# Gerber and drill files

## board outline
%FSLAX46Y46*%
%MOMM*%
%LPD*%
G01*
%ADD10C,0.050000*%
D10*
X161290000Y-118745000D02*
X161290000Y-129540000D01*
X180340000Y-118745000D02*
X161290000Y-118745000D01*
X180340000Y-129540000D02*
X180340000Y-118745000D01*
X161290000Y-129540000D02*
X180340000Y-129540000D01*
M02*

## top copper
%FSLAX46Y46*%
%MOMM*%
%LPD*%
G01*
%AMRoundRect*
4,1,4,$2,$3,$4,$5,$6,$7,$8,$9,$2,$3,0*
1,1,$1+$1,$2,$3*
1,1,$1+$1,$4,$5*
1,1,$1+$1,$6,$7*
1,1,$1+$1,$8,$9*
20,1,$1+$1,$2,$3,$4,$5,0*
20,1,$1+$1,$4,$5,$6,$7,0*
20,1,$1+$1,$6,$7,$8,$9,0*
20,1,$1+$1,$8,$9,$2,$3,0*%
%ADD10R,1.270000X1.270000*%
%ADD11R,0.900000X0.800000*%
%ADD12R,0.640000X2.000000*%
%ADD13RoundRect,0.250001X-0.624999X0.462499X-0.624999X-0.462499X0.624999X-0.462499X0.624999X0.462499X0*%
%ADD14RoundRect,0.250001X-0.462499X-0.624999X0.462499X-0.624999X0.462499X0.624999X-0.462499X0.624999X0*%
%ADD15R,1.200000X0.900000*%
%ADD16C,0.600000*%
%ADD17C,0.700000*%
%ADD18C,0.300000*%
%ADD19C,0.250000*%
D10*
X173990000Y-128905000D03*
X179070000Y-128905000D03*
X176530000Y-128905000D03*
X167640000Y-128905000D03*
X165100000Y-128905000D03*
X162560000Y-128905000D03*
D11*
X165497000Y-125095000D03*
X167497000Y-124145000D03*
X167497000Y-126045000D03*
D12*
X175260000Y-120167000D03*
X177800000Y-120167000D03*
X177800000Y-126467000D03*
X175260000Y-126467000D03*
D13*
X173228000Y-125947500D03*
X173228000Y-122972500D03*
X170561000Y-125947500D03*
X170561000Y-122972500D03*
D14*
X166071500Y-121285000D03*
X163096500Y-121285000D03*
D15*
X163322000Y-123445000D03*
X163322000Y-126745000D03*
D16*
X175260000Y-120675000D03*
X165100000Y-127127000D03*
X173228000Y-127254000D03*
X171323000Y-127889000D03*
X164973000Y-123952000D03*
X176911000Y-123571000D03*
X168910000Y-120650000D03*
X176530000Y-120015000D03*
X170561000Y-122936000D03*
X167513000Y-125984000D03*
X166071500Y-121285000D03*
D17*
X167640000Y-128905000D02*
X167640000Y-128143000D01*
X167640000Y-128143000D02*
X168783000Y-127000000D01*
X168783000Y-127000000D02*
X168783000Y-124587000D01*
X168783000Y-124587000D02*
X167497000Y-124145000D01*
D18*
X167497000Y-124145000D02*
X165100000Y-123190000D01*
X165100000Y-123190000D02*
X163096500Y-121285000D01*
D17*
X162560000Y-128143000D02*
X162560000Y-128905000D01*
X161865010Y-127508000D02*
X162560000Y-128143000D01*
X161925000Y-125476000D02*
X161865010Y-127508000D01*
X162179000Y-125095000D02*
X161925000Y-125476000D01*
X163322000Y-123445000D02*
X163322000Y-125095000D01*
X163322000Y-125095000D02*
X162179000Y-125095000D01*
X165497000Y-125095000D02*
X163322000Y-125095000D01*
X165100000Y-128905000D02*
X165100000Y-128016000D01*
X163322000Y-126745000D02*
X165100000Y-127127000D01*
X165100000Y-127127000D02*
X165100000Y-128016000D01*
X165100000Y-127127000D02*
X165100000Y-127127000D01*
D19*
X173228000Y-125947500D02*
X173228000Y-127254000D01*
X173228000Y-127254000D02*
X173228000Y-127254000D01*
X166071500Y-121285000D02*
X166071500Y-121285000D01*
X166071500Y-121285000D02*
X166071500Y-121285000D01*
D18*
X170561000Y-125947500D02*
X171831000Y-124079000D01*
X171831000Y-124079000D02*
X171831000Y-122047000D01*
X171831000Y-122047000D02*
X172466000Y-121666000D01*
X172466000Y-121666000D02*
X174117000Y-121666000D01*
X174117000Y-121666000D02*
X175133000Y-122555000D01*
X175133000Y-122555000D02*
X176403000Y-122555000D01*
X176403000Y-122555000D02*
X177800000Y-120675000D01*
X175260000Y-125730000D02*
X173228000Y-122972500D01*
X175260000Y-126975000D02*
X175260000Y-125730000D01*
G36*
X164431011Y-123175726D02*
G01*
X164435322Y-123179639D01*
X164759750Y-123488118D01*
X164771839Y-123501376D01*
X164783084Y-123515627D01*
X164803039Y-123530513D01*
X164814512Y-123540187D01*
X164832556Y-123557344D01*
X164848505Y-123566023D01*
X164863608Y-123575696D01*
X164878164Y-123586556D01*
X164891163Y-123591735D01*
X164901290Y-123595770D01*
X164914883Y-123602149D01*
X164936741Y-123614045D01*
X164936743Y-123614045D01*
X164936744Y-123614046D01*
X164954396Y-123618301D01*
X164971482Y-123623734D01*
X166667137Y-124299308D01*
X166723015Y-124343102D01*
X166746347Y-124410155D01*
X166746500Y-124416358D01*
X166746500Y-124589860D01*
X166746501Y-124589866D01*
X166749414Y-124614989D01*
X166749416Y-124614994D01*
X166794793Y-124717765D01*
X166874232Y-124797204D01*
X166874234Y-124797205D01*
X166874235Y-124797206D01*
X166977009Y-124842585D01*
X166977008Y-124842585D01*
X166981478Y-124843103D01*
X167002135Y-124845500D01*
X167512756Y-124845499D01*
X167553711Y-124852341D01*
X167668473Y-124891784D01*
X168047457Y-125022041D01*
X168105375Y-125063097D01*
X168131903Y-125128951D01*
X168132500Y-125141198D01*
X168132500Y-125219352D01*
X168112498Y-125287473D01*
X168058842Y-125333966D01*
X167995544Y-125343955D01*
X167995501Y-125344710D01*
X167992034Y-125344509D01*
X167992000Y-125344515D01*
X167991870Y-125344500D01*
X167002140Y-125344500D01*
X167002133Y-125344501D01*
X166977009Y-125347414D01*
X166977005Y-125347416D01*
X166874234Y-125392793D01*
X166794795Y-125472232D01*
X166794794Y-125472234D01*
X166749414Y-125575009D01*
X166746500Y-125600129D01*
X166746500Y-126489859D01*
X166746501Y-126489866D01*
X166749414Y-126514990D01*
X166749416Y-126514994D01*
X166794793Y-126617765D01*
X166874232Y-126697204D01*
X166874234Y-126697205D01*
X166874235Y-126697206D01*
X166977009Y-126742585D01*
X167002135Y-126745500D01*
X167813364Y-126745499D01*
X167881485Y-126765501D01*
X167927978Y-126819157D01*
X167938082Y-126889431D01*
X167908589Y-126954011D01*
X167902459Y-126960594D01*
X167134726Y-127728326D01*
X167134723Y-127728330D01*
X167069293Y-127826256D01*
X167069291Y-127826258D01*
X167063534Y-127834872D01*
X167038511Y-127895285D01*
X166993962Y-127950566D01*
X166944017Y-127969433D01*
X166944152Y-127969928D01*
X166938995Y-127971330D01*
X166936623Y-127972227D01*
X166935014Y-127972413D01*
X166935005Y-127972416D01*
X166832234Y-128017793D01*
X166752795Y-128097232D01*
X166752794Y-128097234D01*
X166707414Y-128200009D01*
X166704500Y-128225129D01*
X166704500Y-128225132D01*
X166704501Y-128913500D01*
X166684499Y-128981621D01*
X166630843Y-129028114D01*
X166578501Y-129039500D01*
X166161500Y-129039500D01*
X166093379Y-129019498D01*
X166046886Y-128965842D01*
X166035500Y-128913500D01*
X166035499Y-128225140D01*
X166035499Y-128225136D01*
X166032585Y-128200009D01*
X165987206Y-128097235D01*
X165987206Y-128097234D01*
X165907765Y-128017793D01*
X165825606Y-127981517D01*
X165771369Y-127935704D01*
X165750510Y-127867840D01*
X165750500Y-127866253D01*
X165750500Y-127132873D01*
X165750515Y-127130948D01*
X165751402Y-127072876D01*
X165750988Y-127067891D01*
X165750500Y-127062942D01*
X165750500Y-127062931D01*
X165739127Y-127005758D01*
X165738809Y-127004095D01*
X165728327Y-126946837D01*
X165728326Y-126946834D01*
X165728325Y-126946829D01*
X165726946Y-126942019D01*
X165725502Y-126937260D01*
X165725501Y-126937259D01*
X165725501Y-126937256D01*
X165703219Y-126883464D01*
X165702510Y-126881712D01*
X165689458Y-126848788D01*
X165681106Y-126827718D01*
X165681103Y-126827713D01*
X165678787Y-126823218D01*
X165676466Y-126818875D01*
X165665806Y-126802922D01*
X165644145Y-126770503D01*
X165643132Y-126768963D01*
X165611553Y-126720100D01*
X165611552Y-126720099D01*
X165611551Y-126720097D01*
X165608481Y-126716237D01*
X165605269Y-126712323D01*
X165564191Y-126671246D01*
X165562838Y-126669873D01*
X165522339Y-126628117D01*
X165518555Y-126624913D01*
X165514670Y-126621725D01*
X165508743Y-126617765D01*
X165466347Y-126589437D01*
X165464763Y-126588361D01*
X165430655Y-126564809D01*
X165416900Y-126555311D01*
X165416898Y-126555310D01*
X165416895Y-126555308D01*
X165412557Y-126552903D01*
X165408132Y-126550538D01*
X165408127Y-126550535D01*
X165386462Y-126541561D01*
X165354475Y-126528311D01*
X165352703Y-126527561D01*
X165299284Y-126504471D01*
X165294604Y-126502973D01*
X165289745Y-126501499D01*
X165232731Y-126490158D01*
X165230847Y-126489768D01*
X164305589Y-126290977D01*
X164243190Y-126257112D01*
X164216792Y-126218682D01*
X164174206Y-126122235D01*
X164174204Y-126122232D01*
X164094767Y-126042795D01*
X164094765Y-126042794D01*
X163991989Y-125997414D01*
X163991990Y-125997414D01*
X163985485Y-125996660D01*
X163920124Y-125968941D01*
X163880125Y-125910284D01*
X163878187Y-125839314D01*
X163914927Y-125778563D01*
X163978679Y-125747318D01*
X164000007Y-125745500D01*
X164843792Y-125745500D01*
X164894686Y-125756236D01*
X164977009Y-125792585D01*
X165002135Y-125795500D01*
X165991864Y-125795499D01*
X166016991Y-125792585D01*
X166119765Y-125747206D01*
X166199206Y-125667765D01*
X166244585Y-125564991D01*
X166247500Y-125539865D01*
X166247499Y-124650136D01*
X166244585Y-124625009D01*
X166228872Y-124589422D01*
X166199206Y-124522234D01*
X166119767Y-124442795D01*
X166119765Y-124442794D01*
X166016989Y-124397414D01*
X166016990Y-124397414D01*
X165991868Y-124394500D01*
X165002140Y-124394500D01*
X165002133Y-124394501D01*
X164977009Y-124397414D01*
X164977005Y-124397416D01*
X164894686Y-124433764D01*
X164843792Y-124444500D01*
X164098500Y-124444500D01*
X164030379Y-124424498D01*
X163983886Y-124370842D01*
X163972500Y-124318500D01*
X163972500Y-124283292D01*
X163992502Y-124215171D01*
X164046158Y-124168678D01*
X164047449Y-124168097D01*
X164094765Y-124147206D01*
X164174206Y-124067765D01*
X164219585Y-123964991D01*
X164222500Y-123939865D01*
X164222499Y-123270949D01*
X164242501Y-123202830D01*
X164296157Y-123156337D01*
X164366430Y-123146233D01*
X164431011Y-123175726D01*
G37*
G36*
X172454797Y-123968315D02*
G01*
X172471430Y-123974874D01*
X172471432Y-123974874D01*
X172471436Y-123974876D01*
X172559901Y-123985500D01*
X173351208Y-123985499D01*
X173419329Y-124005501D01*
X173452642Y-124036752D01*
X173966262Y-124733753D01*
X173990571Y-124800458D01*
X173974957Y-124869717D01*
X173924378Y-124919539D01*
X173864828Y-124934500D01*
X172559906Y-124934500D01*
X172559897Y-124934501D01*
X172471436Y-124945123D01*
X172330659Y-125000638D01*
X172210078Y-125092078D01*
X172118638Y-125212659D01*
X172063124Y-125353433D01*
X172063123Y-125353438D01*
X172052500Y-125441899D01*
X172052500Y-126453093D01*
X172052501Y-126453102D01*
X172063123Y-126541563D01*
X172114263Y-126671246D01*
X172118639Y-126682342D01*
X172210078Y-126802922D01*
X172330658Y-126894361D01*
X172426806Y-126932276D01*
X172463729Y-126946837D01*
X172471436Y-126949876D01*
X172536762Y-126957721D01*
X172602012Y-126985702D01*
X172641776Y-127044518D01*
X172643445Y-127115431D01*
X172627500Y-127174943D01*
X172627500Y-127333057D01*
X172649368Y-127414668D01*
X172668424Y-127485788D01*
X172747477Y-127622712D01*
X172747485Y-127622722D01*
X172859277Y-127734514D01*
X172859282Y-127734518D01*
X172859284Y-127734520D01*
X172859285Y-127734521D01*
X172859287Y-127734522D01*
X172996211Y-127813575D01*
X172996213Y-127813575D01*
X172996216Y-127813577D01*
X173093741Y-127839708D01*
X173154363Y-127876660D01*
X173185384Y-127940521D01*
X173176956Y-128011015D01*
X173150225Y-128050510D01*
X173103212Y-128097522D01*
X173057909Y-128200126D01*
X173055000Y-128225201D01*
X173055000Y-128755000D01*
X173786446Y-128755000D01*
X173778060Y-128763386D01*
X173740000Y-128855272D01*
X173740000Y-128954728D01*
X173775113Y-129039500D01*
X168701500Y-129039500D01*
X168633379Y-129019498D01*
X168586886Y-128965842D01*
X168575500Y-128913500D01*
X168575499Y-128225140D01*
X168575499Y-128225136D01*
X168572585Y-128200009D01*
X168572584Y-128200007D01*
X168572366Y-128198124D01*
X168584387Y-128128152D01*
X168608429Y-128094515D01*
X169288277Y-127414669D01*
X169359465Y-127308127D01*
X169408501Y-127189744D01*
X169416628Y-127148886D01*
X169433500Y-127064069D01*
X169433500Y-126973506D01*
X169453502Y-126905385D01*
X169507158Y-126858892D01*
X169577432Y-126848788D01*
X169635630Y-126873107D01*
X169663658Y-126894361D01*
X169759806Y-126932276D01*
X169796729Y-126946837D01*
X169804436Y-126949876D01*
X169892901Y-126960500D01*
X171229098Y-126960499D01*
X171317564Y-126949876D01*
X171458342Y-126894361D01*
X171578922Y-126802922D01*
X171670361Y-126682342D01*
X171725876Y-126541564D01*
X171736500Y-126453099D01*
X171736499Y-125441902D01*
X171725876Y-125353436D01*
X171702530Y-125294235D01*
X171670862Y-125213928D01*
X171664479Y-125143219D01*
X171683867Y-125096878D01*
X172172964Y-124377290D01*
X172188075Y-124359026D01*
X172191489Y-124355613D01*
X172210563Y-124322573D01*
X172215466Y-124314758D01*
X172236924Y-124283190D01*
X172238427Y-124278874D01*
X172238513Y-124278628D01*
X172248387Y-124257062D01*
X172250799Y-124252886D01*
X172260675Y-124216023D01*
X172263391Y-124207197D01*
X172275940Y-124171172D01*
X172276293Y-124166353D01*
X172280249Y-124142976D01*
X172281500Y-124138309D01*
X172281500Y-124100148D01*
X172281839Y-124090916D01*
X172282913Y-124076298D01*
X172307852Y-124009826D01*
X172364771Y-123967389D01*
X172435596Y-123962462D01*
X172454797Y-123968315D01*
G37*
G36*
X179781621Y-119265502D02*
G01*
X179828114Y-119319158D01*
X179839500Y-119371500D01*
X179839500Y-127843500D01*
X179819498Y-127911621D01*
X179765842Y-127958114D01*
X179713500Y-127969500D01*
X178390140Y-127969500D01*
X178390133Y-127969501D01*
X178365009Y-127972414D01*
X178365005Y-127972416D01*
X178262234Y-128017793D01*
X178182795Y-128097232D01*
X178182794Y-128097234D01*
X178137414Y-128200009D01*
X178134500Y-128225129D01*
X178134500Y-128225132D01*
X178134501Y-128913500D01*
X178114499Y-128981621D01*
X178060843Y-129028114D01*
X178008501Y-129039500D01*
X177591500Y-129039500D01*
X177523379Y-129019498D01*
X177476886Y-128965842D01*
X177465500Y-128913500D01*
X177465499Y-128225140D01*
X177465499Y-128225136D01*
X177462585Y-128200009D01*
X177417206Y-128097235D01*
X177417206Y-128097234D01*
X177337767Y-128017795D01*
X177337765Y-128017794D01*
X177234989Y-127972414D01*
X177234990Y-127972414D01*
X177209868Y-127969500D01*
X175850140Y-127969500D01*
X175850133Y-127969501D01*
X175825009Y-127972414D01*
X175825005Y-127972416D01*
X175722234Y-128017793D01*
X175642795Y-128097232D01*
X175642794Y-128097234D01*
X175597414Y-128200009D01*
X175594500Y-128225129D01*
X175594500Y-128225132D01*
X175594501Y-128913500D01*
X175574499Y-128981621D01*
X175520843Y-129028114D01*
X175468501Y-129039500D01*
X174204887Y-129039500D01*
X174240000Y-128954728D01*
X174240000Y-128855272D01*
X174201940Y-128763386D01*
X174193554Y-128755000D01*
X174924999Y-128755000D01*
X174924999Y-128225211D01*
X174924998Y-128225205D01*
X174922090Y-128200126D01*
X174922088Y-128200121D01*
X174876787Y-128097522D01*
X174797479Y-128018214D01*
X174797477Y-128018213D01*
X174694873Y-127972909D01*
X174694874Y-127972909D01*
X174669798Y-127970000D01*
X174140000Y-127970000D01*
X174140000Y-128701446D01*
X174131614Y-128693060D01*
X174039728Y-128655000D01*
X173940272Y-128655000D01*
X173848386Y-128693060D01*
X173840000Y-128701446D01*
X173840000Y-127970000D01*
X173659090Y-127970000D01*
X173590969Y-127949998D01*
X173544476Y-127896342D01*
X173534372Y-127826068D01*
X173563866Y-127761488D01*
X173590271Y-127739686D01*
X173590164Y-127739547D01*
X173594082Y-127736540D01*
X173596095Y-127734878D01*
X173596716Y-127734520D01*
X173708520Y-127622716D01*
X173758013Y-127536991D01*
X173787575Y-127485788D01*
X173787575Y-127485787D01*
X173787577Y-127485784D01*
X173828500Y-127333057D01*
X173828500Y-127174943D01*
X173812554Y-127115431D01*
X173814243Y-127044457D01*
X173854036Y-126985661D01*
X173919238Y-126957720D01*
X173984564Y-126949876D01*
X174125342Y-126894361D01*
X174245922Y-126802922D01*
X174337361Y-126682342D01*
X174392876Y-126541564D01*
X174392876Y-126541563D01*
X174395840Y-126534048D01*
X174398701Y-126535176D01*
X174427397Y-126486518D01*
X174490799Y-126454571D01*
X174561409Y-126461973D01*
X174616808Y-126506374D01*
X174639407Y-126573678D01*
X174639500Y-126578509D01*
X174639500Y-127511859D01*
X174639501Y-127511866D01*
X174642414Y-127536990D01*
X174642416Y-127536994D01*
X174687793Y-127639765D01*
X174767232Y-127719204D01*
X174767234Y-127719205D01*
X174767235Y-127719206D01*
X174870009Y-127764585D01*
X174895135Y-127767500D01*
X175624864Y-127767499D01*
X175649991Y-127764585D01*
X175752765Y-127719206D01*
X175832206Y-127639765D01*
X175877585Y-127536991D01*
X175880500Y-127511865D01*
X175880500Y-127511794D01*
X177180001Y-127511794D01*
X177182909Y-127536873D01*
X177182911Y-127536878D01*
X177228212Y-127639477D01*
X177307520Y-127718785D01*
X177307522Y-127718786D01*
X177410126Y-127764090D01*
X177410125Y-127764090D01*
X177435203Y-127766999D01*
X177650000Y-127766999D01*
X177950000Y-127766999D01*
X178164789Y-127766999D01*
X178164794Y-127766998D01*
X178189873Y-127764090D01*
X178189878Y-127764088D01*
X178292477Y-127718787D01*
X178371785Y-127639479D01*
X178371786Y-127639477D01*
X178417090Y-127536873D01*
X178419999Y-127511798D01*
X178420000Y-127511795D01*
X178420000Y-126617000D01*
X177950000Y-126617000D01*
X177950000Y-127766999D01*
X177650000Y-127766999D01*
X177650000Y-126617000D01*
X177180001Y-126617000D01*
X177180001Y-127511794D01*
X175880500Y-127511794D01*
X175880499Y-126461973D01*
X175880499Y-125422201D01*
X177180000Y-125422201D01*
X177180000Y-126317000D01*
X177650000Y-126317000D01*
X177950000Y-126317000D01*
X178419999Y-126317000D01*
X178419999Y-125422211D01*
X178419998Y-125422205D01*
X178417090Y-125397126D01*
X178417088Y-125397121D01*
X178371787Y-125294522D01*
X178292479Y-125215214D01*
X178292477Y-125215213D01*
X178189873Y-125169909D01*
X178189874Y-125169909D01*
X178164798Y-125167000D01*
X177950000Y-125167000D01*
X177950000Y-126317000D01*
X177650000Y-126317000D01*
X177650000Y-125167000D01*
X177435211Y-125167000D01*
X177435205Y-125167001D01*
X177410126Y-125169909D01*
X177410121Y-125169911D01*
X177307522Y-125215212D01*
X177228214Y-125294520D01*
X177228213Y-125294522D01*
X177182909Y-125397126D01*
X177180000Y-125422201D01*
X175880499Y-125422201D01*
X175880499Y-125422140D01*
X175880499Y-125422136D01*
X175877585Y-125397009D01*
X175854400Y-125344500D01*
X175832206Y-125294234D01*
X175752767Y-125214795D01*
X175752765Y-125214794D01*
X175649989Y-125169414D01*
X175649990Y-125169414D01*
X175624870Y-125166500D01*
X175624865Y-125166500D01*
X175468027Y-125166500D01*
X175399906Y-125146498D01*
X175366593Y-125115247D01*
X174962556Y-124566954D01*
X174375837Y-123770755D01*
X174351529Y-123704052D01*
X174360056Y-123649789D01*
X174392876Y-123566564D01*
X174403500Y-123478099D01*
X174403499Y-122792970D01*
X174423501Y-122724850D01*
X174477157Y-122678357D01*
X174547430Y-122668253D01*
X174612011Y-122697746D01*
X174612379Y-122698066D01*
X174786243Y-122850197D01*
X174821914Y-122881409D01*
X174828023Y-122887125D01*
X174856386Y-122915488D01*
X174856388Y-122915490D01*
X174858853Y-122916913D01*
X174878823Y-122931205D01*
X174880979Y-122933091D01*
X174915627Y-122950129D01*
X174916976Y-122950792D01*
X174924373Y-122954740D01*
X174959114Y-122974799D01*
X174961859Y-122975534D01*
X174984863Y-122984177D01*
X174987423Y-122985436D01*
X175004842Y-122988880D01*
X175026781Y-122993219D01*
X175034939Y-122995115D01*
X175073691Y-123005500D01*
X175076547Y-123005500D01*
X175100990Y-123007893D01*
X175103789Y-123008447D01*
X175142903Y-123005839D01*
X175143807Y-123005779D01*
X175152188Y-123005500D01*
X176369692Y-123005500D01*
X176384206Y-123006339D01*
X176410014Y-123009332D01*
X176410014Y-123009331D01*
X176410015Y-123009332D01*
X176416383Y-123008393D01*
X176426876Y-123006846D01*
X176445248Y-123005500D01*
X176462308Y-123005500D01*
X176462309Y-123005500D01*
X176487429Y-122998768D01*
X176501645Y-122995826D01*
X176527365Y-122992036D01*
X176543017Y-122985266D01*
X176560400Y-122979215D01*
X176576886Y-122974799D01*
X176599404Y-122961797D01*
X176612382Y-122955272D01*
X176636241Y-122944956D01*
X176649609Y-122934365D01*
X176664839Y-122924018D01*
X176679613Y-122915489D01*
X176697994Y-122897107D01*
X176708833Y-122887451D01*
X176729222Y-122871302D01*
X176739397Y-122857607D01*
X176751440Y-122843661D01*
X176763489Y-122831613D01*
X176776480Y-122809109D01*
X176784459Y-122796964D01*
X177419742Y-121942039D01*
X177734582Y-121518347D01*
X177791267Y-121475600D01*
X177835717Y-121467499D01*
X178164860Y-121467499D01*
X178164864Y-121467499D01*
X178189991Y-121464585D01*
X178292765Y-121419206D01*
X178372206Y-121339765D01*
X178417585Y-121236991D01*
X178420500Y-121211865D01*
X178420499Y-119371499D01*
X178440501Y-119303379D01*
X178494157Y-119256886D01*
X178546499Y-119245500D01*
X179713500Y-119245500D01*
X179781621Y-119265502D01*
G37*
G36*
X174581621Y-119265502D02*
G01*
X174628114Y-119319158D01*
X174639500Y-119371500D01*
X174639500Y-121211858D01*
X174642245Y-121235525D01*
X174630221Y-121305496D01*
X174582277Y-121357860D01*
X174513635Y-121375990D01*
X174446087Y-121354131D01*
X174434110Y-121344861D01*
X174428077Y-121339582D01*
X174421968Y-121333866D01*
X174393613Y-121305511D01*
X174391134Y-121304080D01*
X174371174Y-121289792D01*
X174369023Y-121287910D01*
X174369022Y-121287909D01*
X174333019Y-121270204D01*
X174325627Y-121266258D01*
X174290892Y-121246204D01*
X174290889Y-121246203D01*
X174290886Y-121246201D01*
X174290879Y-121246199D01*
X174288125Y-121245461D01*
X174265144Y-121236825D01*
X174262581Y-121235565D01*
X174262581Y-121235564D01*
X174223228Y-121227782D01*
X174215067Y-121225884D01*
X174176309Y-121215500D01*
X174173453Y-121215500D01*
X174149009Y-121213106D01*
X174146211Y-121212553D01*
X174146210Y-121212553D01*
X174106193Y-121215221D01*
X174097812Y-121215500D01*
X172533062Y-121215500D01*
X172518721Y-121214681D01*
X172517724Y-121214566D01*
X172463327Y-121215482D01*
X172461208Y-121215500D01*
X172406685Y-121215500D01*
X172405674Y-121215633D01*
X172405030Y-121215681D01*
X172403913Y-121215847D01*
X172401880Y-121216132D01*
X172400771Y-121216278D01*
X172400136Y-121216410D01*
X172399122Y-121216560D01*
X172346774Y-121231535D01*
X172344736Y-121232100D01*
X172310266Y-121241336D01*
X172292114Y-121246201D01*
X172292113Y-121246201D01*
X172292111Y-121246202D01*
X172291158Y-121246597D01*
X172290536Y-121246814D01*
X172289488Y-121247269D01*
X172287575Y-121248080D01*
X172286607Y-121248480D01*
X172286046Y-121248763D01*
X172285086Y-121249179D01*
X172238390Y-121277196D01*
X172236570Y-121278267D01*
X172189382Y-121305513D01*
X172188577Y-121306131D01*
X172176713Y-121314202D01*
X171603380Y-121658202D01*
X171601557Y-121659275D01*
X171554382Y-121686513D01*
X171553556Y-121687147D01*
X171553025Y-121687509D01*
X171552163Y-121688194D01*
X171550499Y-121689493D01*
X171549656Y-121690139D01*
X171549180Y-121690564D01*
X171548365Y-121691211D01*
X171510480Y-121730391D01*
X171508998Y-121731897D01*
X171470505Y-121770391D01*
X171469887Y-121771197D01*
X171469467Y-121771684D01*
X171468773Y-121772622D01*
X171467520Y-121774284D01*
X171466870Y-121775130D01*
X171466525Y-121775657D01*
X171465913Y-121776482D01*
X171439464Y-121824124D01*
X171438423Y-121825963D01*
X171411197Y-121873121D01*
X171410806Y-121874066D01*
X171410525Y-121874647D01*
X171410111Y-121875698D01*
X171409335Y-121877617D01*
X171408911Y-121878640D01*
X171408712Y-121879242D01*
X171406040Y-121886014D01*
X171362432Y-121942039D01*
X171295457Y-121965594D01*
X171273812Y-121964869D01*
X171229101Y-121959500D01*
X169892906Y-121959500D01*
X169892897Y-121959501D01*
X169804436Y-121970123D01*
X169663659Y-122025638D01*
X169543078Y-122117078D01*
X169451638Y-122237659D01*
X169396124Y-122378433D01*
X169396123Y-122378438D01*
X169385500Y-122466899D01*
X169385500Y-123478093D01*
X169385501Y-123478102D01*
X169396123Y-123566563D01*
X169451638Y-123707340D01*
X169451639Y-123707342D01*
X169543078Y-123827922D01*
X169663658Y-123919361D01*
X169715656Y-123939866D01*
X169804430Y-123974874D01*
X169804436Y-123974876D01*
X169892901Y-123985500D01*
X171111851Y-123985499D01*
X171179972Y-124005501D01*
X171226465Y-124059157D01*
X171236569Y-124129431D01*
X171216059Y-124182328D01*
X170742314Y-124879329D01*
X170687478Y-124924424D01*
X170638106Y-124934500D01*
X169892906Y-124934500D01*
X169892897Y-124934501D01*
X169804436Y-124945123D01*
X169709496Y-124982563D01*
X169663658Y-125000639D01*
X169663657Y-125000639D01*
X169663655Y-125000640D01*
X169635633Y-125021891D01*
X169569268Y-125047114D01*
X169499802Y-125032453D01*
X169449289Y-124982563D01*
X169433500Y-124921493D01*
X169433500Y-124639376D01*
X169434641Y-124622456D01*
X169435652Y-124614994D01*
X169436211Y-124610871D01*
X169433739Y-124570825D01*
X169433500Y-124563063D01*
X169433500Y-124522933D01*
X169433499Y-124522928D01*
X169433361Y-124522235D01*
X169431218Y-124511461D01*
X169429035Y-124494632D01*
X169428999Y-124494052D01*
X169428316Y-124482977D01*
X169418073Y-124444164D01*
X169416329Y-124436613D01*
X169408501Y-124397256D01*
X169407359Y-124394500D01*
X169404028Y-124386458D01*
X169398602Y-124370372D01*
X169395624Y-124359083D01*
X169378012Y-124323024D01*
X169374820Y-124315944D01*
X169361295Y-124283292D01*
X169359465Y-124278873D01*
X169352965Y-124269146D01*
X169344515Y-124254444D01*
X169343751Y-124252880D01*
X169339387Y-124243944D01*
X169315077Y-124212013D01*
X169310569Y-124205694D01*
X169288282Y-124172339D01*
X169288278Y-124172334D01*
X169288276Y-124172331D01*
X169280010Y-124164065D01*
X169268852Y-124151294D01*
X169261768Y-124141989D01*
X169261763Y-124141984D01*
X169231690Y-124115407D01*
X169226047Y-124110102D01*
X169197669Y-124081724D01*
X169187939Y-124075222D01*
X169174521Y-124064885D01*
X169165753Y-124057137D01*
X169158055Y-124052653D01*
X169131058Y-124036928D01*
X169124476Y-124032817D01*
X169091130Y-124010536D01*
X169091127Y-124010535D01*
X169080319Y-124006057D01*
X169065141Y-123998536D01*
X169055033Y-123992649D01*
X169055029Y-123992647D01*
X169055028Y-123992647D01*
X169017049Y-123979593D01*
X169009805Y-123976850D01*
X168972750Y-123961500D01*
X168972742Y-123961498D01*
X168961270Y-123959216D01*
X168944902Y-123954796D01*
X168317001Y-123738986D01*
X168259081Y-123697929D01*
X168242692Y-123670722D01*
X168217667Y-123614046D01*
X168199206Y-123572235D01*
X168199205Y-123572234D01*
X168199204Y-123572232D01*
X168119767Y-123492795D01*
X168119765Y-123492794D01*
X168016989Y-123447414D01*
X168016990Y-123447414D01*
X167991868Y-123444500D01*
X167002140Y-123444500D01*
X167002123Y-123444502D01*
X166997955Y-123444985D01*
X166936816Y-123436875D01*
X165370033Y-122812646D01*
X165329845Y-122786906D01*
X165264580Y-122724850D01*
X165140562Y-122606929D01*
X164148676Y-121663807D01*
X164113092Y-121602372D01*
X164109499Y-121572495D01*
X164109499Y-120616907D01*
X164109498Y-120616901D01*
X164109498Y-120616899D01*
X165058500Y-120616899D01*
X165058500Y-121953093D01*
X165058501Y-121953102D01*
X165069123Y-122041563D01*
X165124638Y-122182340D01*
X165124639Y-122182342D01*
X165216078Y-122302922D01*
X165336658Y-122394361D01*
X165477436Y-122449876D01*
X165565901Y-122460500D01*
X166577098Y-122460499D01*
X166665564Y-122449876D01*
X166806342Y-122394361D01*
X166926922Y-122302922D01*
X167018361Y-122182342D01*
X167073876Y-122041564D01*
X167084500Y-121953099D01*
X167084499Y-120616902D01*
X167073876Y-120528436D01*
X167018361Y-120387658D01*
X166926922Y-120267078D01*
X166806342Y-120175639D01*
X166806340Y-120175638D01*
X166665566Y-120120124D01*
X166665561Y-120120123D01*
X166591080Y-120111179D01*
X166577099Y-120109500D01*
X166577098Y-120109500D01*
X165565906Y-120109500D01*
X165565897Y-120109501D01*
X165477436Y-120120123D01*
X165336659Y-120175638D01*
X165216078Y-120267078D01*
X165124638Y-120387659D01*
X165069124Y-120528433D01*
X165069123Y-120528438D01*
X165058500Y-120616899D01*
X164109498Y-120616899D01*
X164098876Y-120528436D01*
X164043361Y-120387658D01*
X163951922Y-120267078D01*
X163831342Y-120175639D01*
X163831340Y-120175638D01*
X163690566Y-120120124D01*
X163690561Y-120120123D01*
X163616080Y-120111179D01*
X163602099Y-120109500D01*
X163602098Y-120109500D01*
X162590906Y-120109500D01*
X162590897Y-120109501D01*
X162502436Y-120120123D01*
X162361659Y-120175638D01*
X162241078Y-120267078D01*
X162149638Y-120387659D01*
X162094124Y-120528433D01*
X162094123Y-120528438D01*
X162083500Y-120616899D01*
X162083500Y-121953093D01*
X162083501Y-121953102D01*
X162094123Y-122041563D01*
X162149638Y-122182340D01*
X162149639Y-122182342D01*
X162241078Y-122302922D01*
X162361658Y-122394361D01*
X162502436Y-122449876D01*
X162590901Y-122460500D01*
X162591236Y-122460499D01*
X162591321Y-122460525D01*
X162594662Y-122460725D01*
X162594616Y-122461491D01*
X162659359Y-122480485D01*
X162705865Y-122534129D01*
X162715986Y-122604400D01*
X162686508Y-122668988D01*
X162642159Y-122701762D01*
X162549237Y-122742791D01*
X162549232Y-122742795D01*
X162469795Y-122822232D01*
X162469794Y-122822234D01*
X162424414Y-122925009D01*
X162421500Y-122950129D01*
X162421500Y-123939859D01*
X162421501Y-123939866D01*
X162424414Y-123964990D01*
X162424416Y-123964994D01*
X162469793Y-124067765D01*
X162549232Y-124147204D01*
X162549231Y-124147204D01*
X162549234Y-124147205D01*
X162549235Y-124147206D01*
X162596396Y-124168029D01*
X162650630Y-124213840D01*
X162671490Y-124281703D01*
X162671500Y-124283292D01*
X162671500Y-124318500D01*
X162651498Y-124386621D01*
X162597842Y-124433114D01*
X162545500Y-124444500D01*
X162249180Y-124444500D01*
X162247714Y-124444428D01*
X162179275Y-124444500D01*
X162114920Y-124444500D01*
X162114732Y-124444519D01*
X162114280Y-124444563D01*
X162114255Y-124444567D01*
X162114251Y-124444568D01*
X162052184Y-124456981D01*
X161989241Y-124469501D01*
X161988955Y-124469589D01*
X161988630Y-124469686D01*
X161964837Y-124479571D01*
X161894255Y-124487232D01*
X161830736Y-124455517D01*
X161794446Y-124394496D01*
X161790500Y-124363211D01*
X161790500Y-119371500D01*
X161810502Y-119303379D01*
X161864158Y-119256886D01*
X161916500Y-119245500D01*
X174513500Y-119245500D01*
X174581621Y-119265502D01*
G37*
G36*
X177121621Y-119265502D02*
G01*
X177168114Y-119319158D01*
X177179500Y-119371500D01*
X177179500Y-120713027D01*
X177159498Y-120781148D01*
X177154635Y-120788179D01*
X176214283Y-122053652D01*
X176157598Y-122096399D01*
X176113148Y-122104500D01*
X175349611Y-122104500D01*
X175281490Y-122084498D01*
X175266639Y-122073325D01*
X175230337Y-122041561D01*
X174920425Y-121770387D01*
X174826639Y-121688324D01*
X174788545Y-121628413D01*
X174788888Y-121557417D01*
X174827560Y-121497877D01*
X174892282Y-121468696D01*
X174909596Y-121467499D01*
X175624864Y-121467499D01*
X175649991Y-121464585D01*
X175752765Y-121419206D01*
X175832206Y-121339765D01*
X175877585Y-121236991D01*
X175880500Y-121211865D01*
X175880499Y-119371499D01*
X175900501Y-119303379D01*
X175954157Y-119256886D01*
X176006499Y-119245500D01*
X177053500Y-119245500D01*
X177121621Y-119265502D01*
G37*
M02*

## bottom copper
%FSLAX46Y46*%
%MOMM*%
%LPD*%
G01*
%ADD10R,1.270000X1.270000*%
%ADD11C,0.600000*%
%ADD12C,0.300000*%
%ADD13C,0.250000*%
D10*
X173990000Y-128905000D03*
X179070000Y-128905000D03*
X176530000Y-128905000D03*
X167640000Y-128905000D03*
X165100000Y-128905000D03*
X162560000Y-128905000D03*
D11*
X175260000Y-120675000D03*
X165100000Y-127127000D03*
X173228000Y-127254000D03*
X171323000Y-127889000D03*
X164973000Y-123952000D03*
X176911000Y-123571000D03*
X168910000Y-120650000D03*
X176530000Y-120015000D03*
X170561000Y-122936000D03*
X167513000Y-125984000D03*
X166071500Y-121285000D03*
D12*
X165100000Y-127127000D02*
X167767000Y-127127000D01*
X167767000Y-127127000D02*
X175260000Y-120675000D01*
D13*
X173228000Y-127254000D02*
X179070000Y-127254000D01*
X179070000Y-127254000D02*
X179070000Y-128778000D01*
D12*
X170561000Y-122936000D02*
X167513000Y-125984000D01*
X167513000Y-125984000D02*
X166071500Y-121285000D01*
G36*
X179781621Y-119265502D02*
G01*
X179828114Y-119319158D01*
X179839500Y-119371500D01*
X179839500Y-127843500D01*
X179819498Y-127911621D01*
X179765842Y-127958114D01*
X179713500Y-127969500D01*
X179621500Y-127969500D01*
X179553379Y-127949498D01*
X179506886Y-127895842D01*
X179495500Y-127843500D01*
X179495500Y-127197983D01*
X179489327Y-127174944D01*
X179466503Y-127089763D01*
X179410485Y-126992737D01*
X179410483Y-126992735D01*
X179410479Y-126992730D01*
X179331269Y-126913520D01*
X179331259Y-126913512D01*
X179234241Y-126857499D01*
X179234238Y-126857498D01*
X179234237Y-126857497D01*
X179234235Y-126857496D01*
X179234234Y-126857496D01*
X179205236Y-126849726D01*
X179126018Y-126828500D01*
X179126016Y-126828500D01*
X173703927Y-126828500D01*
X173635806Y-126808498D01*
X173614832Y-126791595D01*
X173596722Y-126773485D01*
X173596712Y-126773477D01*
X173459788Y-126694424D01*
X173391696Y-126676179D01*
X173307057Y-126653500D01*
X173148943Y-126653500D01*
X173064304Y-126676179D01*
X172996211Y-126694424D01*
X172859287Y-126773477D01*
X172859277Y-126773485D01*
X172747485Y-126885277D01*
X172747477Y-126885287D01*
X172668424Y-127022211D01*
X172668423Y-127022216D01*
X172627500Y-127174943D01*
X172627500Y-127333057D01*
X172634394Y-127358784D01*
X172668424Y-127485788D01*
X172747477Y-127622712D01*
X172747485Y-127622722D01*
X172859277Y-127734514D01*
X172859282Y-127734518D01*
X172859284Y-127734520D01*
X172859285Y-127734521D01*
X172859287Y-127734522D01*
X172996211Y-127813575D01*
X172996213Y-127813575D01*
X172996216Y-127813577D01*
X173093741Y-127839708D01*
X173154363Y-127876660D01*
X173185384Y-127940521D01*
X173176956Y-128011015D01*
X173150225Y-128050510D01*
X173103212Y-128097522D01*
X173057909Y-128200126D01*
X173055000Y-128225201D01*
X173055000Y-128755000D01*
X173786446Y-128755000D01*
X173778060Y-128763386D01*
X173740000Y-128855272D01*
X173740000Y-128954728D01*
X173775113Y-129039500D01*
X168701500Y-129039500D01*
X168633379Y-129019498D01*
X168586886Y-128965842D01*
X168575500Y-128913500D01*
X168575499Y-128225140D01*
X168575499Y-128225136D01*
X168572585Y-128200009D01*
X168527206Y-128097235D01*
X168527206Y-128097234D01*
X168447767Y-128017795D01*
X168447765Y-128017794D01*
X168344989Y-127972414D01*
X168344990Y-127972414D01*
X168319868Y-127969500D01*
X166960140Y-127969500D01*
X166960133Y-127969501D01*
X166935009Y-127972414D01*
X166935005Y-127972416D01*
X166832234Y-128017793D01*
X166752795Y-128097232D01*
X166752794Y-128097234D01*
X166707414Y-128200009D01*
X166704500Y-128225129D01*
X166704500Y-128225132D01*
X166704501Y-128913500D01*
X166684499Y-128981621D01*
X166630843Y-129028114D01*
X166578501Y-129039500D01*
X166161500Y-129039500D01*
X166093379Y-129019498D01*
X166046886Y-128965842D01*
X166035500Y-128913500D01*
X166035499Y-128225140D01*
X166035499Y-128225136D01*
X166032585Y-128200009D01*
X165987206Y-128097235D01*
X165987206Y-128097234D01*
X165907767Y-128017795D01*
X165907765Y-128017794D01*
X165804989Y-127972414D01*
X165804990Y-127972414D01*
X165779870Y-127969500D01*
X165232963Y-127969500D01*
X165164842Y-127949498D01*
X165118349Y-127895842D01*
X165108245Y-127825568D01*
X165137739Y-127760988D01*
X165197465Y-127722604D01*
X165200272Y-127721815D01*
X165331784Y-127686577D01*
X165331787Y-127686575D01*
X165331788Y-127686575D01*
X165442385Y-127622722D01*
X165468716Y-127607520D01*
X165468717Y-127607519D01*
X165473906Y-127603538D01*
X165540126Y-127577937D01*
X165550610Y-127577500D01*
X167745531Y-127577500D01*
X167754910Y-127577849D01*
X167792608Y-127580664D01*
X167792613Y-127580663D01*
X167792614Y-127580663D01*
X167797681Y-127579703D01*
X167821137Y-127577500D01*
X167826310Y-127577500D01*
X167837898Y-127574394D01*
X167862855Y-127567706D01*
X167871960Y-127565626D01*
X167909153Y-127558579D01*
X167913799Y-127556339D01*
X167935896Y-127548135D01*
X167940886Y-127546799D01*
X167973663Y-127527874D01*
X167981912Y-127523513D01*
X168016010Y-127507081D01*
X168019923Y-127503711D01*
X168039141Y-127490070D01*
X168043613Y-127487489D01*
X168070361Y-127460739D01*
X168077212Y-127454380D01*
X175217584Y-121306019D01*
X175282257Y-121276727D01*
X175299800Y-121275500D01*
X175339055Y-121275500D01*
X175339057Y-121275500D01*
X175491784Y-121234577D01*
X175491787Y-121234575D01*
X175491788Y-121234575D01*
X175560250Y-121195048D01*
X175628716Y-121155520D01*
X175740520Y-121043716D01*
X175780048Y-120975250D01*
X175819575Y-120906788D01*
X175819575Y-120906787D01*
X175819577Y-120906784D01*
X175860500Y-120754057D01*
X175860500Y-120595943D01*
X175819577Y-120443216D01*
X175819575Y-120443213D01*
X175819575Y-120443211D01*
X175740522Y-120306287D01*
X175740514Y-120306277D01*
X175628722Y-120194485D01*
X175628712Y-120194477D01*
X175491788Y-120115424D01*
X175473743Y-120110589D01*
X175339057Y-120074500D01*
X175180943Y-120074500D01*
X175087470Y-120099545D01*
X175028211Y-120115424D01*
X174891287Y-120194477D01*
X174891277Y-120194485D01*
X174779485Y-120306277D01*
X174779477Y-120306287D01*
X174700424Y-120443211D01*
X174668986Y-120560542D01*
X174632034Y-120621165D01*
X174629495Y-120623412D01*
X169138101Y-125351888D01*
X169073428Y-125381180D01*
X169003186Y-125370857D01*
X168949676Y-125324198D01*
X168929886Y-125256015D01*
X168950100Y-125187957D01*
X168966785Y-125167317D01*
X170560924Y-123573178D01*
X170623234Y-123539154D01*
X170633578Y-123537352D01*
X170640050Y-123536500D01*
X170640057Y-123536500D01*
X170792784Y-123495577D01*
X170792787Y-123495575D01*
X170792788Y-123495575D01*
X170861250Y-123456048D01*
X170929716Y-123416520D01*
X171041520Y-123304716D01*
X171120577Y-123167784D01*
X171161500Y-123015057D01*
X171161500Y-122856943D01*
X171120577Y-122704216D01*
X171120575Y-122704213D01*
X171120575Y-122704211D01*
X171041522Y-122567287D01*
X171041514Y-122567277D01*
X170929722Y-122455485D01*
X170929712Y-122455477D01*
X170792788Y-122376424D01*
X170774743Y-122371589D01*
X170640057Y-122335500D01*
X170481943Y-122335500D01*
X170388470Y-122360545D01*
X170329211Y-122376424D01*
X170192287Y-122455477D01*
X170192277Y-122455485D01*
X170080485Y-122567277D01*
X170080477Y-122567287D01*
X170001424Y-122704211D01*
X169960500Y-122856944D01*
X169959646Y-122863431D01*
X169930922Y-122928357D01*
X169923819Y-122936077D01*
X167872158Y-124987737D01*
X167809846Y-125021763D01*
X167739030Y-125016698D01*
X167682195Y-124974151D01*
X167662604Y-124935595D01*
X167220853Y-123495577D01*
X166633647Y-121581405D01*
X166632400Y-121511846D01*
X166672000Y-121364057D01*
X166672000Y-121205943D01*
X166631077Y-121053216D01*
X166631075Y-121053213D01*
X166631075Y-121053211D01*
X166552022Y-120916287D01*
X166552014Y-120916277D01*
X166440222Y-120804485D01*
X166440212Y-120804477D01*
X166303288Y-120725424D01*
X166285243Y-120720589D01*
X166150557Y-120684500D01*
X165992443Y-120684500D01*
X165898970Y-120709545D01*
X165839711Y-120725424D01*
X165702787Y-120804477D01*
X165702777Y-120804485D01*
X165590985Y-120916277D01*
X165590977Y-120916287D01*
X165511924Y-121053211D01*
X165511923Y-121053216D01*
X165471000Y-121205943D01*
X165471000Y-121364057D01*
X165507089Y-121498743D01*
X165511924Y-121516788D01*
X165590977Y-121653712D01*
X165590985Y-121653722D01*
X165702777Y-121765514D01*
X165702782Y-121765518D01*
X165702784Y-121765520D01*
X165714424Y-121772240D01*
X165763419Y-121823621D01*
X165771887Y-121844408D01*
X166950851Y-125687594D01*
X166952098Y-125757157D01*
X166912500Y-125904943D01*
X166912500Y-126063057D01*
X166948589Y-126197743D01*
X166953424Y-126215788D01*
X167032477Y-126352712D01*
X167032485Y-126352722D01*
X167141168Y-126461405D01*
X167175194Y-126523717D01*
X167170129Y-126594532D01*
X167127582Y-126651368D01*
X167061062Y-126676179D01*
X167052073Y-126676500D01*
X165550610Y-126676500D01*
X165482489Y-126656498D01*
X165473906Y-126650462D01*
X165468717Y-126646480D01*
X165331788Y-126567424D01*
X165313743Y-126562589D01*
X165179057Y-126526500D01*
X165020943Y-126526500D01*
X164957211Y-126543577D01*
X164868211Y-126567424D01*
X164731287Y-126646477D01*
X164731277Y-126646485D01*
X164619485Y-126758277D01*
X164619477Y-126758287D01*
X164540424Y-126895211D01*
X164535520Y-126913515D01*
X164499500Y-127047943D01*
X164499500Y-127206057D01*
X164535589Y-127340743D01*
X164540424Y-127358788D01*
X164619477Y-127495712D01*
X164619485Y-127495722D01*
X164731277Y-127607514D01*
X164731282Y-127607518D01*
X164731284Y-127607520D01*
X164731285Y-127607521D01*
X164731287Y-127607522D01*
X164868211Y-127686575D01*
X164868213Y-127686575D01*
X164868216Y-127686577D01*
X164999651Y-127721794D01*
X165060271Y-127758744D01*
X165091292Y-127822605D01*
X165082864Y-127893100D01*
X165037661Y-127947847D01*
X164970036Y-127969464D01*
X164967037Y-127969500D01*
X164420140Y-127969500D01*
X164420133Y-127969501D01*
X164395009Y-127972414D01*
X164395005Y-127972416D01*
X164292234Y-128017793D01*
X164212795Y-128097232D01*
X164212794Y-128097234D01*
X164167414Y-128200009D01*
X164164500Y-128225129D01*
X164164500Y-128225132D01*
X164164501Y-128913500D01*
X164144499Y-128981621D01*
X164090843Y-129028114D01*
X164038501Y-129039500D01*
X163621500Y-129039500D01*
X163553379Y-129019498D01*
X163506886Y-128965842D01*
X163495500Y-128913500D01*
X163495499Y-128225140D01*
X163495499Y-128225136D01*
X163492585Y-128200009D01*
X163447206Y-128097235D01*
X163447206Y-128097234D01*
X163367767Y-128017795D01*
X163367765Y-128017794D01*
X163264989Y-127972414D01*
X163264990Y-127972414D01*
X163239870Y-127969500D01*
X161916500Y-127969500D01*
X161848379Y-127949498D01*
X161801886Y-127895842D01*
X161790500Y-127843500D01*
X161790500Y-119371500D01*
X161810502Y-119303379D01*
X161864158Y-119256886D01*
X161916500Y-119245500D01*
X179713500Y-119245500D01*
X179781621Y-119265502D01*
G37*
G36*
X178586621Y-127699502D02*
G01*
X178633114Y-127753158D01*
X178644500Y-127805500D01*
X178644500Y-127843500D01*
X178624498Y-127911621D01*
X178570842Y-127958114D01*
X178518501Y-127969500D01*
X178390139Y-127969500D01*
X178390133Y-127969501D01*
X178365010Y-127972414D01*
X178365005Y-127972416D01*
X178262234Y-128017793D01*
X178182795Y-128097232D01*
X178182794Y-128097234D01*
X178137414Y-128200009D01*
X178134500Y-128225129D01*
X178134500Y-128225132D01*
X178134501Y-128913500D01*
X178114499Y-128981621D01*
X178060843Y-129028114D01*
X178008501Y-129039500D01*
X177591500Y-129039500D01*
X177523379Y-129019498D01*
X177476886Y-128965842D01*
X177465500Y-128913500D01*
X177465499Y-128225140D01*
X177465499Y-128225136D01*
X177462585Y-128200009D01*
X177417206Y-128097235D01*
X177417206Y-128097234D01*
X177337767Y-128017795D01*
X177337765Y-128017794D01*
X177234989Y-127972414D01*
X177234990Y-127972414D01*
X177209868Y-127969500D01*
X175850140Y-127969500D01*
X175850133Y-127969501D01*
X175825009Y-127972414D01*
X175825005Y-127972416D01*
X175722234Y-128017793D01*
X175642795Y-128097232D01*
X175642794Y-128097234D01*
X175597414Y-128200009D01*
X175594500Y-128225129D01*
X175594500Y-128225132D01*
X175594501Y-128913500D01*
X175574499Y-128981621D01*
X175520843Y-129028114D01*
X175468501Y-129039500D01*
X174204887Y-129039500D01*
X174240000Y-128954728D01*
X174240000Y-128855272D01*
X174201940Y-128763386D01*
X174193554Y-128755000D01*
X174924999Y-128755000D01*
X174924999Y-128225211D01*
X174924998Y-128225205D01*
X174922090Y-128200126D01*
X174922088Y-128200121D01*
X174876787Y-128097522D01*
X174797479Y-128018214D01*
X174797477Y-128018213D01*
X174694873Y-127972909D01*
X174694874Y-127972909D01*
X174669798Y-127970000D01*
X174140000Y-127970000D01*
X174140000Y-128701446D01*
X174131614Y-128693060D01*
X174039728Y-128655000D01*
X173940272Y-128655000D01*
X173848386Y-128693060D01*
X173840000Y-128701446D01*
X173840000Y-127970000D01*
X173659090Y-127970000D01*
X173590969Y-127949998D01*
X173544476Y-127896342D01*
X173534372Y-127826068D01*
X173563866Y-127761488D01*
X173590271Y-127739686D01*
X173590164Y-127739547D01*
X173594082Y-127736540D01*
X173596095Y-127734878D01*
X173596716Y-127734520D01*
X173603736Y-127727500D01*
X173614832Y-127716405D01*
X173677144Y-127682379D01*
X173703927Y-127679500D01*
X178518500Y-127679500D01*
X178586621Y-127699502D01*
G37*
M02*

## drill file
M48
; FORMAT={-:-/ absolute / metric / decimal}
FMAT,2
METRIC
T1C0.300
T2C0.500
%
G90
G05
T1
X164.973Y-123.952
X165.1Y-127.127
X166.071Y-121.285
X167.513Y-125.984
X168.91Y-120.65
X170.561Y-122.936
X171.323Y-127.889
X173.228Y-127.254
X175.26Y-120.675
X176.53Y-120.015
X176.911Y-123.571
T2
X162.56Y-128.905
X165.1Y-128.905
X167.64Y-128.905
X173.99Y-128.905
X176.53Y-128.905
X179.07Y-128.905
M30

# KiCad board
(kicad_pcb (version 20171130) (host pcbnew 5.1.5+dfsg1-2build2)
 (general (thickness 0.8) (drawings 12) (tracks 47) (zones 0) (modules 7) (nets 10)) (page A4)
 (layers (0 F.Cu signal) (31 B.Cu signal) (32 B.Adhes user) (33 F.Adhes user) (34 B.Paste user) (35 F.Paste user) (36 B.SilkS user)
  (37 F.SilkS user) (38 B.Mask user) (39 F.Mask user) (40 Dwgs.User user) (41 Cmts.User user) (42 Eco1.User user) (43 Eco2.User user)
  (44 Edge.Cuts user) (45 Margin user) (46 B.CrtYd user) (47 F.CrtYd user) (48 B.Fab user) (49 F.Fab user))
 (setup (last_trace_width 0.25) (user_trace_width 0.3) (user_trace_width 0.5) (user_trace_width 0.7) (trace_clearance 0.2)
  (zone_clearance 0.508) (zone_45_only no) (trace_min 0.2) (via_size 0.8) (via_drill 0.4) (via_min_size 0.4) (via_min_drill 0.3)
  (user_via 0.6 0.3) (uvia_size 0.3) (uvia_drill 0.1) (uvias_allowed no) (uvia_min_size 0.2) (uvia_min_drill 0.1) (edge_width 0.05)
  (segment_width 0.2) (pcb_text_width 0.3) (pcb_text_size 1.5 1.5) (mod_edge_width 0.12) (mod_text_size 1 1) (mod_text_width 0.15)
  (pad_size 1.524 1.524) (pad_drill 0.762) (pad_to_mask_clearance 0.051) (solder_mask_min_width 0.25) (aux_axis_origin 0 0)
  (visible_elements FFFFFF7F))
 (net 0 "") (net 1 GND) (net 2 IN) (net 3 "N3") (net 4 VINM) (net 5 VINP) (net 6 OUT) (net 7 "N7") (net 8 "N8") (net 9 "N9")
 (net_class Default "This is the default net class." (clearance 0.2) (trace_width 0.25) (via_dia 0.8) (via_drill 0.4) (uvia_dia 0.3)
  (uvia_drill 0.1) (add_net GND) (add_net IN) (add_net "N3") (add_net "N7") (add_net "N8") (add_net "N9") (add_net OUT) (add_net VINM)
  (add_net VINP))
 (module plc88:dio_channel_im (layer F.Cu) (at 169.545 126.365)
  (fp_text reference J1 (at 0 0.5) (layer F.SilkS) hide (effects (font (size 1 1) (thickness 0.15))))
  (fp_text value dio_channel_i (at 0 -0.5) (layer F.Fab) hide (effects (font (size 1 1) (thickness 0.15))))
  (pad 4 thru_hole rect (at 4.445 2.54) (size 1.27 1.27) (drill 0.5) (layers *.Cu *.Mask) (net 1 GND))
  (pad 6 thru_hole rect (at 9.525 2.54) (size 1.27 1.27) (drill 0.5) (layers *.Cu *.Mask) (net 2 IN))
  (pad 5 thru_hole rect (at 6.985 2.54) (size 1.27 1.27) (drill 0.5) (layers *.Cu *.Mask) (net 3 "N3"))
  (pad 3 thru_hole rect (at -1.905 2.54) (size 1.27 1.27) (drill 0.5) (layers *.Cu *.Mask) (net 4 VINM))
  (pad 2 thru_hole rect (at -4.445 2.54) (size 1.27 1.27) (drill 0.5) (layers *.Cu *.Mask) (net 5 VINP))
  (pad 1 thru_hole rect (at -6.985 2.54) (size 1.27 1.27) (drill 0.5) (layers *.Cu *.Mask) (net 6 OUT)))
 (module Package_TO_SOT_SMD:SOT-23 (layer F.Cu) (at 166.497 125.095 180)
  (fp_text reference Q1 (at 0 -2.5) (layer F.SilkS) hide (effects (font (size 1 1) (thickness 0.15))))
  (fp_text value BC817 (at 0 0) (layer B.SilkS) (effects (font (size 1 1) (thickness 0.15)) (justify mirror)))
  (pad 3 smd rect (at 1 0 180) (size 0.9 0.8) (layers F.Cu F.Paste F.Mask) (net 6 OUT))
  (pad 2 smd rect (at -1 0.95 180) (size 0.9 0.8) (layers F.Cu F.Paste F.Mask) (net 4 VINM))
  (pad 1 smd rect (at -1 -0.95 180) (size 0.9 0.8) (layers F.Cu F.Paste F.Mask) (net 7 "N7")))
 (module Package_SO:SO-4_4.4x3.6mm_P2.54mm (layer F.Cu) (at 176.53 123.317 90)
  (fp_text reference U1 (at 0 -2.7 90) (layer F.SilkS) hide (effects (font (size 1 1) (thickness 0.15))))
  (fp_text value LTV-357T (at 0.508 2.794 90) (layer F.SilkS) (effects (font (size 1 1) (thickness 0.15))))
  (pad 4 smd rect (at 3.15 -1.27 90) (size 2 0.64) (layers F.Cu F.Paste F.Mask) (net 5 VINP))
  (pad 3 smd rect (at 3.15 1.27 90) (size 2 0.64) (layers F.Cu F.Paste F.Mask) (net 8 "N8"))
  (pad 2 smd rect (at -3.15 1.27 90) (size 2 0.64) (layers F.Cu F.Paste F.Mask) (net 1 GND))
  (pad 1 smd rect (at -3.15 -1.27 90) (size 2 0.64) (layers F.Cu F.Paste F.Mask) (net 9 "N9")))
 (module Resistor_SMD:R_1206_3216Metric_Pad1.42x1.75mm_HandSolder (layer F.Cu) (at 173.228 124.46 270)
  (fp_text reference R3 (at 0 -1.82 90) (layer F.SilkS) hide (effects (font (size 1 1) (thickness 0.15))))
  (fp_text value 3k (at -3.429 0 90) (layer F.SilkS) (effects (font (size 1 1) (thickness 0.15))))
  (pad 2 smd roundrect (at 1.4875 0 270) (size 1.425 1.75) (layers F.Cu F.Paste F.Mask) (roundrect_rratio 0.175439) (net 2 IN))
  (pad 1 smd roundrect (at -1.4875 0 270) (size 1.425 1.75) (layers F.Cu F.Paste F.Mask) (roundrect_rratio 0.175439) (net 9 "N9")))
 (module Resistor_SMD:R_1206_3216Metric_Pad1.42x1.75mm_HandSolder (layer F.Cu) (at 170.561 124.46 270)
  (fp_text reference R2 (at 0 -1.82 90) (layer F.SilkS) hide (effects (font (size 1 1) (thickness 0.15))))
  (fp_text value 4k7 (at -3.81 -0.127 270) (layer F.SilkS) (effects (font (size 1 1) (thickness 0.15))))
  (pad 2 smd roundrect (at 1.4875 0 270) (size 1.425 1.75) (layers F.Cu F.Paste F.Mask) (roundrect_rratio 0.175439) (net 8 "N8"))
  (pad 1 smd roundrect (at -1.4875 0 270) (size 1.425 1.75) (layers F.Cu F.Paste F.Mask) (roundrect_rratio 0.175439) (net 7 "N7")))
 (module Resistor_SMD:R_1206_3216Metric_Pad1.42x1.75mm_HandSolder (layer F.Cu) (at 164.584 121.285)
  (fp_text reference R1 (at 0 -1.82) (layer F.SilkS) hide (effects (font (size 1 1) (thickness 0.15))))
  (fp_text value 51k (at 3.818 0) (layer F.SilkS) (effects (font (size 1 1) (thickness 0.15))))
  (pad 2 smd roundrect (at 1.4875 0) (size 1.425 1.75) (layers F.Cu F.Paste F.Mask) (roundrect_rratio 0.175439) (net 7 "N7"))
  (pad 1 smd roundrect (at -1.4875 0) (size 1.425 1.75) (layers F.Cu F.Paste F.Mask) (roundrect_rratio 0.175439) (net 4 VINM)))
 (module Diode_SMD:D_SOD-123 (layer F.Cu) (at 163.322 125.095 90)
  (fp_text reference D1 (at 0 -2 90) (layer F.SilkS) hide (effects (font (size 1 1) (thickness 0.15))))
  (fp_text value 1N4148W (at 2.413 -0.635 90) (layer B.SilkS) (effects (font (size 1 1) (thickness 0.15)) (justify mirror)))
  (pad 2 smd rect (at 1.65 0 90) (size 0.9 1.2) (layers F.Cu F.Paste F.Mask) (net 6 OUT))
  (pad 1 smd rect (at -1.65 0 90) (size 0.9 1.2) (layers F.Cu F.Paste F.Mask) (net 5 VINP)))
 (gr_line (start 161.29 118.745) (end 161.29 129.54) (layer Edge.Cuts) (width 0.05))
 (gr_line (start 180.34 118.745) (end 161.29 118.745) (layer Edge.Cuts) (width 0.05))
 (gr_line (start 180.34 129.54) (end 180.34 118.745) (layer Edge.Cuts) (width 0.05))
 (gr_line (start 161.29 129.54) (end 180.34 129.54) (layer Edge.Cuts) (width 0.05))
 (segment (start 167.64 128.905) (end 167.64 128.143) (width 0.7) (layer F.Cu) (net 4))
 (segment (start 167.64 128.143) (end 168.783 127) (width 0.7) (layer F.Cu) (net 4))
 (segment (start 168.783 127) (end 168.783 124.587) (width 0.7) (layer F.Cu) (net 4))
 (segment (start 168.783 124.587) (end 167.497 124.145) (width 0.7) (layer F.Cu) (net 4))
 (segment (start 167.497 124.145) (end 165.1 123.19) (width 0.3) (layer F.Cu) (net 4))
 (segment (start 165.1 123.19) (end 163.0965 121.285) (width 0.3) (layer F.Cu) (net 4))
 (segment (start 162.56 128.143) (end 162.56 128.905) (width 0.7) (layer F.Cu) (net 6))
 (segment (start 161.86501 127.508) (end 162.56 128.143) (width 0.7) (layer F.Cu) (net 6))
 (segment (start 161.925 125.476) (end 161.86501 127.508) (width 0.7) (layer F.Cu) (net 6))
 (segment (start 162.179 125.095) (end 161.925 125.476) (width 0.7) (layer F.Cu) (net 6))
 (segment (start 163.322 123.445) (end 163.322 125.095) (width 0.7) (layer F.Cu) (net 6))
 (segment (start 163.322 125.095) (end 162.179 125.095) (width 0.7) (layer F.Cu) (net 6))
 (segment (start 165.497 125.095) (end 163.322 125.095) (width 0.7) (layer F.Cu) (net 6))
 (segment (start 165.1 128.905) (end 165.1 128.016) (width 0.7) (layer F.Cu) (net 5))
 (via (at 175.26 120.675) (size 0.6) (drill 0.3) (layers F.Cu B.Cu) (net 5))
 (segment (start 163.322 126.745) (end 165.1 127.127) (width 0.7) (layer F.Cu) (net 5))
 (segment (start 165.1 127.127) (end 165.1 128.016) (width 0.7) (layer F.Cu) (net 5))
 (segment (start 165.1 127.127) (end 165.1 127.127) (width 0.7) (layer F.Cu) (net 5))
 (via (at 165.1 127.127) (size 0.6) (drill 0.3) (layers F.Cu B.Cu) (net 5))
 (segment (start 165.1 127.127) (end 167.767 127.127) (width 0.3) (layer B.Cu) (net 5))
 (segment (start 167.767 127.127) (end 175.26 120.675) (width 0.3) (layer B.Cu) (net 5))
 (segment (start 173.228 125.9475) (end 173.228 127.254) (width 0.25) (layer F.Cu) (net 2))
 (segment (start 173.228 127.254) (end 173.228 127.254) (width 0.25) (layer F.Cu) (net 2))
 (via (at 173.228 127.254) (size 0.6) (drill 0.3) (layers F.Cu B.Cu) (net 2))
 (segment (start 173.228 127.254) (end 179.07 127.254) (width 0.25) (layer B.Cu) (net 2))
 (segment (start 179.07 127.254) (end 179.07 128.778) (width 0.25) (layer B.Cu) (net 2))
 (via (at 171.323 127.889) (size 0.6) (drill 0.3) (layers F.Cu B.Cu) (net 1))
 (via (at 164.973 123.952) (size 0.6) (drill 0.3) (layers F.Cu B.Cu) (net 1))
 (via (at 176.911 123.571) (size 0.6) (drill 0.3) (layers F.Cu B.Cu) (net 1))
 (via (at 168.91 120.65) (size 0.6) (drill 0.3) (layers F.Cu B.Cu) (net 1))
 (via (at 176.53 120.015) (size 0.6) (drill 0.3) (layers F.Cu B.Cu) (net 1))
 (via (at 170.561 122.936) (size 0.6) (drill 0.3) (layers F.Cu B.Cu) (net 7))
 (via (at 167.513 125.984) (size 0.6) (drill 0.3) (layers F.Cu B.Cu) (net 7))
 (segment (start 166.0715 121.285) (end 166.0715 121.285) (width 0.25) (layer F.Cu) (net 7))
 (segment (start 166.0715 121.285) (end 166.0715 121.285) (width 0.25) (layer F.Cu) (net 7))
 (via (at 166.0715 121.285) (size 0.6) (drill 0.3) (layers F.Cu B.Cu) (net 7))
 (segment (start 170.561 122.936) (end 167.513 125.984) (width 0.3) (layer B.Cu) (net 7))
 (segment (start 167.513 125.984) (end 166.0715 121.285) (width 0.3) (layer B.Cu) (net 7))
 (segment (start 170.561 125.9475) (end 171.831 124.079) (width 0.3) (layer F.Cu) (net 8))
 (segment (start 171.831 124.079) (end 171.831 122.047) (width 0.3) (layer F.Cu) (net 8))
 (segment (start 171.831 122.047) (end 172.466 121.666) (width 0.3) (layer F.Cu) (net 8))
 (segment (start 172.466 121.666) (end 174.117 121.666) (width 0.3) (layer F.Cu) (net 8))
 (segment (start 174.117 121.666) (end 175.133 122.555) (width 0.3) (layer F.Cu) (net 8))
 (segment (start 175.133 122.555) (end 176.403 122.555) (width 0.3) (layer F.Cu) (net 8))
 (segment (start 176.403 122.555) (end 177.8 120.675) (width 0.3) (layer F.Cu) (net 8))
 (segment (start 175.26 125.73) (end 173.228 122.9725) (width 0.3) (layer F.Cu) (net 9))
 (segment (start 175.26 126.975) (end 175.26 125.73) (width 0.3) (layer F.Cu) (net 9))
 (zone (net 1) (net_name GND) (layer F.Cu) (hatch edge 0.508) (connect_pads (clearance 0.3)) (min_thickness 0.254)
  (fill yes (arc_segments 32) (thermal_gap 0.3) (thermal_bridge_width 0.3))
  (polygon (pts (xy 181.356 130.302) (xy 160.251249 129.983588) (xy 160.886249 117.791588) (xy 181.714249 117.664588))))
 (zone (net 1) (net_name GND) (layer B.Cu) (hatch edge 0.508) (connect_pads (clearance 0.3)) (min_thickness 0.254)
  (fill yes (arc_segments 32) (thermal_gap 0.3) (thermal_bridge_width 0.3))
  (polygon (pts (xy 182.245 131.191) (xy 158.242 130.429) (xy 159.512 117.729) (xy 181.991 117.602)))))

